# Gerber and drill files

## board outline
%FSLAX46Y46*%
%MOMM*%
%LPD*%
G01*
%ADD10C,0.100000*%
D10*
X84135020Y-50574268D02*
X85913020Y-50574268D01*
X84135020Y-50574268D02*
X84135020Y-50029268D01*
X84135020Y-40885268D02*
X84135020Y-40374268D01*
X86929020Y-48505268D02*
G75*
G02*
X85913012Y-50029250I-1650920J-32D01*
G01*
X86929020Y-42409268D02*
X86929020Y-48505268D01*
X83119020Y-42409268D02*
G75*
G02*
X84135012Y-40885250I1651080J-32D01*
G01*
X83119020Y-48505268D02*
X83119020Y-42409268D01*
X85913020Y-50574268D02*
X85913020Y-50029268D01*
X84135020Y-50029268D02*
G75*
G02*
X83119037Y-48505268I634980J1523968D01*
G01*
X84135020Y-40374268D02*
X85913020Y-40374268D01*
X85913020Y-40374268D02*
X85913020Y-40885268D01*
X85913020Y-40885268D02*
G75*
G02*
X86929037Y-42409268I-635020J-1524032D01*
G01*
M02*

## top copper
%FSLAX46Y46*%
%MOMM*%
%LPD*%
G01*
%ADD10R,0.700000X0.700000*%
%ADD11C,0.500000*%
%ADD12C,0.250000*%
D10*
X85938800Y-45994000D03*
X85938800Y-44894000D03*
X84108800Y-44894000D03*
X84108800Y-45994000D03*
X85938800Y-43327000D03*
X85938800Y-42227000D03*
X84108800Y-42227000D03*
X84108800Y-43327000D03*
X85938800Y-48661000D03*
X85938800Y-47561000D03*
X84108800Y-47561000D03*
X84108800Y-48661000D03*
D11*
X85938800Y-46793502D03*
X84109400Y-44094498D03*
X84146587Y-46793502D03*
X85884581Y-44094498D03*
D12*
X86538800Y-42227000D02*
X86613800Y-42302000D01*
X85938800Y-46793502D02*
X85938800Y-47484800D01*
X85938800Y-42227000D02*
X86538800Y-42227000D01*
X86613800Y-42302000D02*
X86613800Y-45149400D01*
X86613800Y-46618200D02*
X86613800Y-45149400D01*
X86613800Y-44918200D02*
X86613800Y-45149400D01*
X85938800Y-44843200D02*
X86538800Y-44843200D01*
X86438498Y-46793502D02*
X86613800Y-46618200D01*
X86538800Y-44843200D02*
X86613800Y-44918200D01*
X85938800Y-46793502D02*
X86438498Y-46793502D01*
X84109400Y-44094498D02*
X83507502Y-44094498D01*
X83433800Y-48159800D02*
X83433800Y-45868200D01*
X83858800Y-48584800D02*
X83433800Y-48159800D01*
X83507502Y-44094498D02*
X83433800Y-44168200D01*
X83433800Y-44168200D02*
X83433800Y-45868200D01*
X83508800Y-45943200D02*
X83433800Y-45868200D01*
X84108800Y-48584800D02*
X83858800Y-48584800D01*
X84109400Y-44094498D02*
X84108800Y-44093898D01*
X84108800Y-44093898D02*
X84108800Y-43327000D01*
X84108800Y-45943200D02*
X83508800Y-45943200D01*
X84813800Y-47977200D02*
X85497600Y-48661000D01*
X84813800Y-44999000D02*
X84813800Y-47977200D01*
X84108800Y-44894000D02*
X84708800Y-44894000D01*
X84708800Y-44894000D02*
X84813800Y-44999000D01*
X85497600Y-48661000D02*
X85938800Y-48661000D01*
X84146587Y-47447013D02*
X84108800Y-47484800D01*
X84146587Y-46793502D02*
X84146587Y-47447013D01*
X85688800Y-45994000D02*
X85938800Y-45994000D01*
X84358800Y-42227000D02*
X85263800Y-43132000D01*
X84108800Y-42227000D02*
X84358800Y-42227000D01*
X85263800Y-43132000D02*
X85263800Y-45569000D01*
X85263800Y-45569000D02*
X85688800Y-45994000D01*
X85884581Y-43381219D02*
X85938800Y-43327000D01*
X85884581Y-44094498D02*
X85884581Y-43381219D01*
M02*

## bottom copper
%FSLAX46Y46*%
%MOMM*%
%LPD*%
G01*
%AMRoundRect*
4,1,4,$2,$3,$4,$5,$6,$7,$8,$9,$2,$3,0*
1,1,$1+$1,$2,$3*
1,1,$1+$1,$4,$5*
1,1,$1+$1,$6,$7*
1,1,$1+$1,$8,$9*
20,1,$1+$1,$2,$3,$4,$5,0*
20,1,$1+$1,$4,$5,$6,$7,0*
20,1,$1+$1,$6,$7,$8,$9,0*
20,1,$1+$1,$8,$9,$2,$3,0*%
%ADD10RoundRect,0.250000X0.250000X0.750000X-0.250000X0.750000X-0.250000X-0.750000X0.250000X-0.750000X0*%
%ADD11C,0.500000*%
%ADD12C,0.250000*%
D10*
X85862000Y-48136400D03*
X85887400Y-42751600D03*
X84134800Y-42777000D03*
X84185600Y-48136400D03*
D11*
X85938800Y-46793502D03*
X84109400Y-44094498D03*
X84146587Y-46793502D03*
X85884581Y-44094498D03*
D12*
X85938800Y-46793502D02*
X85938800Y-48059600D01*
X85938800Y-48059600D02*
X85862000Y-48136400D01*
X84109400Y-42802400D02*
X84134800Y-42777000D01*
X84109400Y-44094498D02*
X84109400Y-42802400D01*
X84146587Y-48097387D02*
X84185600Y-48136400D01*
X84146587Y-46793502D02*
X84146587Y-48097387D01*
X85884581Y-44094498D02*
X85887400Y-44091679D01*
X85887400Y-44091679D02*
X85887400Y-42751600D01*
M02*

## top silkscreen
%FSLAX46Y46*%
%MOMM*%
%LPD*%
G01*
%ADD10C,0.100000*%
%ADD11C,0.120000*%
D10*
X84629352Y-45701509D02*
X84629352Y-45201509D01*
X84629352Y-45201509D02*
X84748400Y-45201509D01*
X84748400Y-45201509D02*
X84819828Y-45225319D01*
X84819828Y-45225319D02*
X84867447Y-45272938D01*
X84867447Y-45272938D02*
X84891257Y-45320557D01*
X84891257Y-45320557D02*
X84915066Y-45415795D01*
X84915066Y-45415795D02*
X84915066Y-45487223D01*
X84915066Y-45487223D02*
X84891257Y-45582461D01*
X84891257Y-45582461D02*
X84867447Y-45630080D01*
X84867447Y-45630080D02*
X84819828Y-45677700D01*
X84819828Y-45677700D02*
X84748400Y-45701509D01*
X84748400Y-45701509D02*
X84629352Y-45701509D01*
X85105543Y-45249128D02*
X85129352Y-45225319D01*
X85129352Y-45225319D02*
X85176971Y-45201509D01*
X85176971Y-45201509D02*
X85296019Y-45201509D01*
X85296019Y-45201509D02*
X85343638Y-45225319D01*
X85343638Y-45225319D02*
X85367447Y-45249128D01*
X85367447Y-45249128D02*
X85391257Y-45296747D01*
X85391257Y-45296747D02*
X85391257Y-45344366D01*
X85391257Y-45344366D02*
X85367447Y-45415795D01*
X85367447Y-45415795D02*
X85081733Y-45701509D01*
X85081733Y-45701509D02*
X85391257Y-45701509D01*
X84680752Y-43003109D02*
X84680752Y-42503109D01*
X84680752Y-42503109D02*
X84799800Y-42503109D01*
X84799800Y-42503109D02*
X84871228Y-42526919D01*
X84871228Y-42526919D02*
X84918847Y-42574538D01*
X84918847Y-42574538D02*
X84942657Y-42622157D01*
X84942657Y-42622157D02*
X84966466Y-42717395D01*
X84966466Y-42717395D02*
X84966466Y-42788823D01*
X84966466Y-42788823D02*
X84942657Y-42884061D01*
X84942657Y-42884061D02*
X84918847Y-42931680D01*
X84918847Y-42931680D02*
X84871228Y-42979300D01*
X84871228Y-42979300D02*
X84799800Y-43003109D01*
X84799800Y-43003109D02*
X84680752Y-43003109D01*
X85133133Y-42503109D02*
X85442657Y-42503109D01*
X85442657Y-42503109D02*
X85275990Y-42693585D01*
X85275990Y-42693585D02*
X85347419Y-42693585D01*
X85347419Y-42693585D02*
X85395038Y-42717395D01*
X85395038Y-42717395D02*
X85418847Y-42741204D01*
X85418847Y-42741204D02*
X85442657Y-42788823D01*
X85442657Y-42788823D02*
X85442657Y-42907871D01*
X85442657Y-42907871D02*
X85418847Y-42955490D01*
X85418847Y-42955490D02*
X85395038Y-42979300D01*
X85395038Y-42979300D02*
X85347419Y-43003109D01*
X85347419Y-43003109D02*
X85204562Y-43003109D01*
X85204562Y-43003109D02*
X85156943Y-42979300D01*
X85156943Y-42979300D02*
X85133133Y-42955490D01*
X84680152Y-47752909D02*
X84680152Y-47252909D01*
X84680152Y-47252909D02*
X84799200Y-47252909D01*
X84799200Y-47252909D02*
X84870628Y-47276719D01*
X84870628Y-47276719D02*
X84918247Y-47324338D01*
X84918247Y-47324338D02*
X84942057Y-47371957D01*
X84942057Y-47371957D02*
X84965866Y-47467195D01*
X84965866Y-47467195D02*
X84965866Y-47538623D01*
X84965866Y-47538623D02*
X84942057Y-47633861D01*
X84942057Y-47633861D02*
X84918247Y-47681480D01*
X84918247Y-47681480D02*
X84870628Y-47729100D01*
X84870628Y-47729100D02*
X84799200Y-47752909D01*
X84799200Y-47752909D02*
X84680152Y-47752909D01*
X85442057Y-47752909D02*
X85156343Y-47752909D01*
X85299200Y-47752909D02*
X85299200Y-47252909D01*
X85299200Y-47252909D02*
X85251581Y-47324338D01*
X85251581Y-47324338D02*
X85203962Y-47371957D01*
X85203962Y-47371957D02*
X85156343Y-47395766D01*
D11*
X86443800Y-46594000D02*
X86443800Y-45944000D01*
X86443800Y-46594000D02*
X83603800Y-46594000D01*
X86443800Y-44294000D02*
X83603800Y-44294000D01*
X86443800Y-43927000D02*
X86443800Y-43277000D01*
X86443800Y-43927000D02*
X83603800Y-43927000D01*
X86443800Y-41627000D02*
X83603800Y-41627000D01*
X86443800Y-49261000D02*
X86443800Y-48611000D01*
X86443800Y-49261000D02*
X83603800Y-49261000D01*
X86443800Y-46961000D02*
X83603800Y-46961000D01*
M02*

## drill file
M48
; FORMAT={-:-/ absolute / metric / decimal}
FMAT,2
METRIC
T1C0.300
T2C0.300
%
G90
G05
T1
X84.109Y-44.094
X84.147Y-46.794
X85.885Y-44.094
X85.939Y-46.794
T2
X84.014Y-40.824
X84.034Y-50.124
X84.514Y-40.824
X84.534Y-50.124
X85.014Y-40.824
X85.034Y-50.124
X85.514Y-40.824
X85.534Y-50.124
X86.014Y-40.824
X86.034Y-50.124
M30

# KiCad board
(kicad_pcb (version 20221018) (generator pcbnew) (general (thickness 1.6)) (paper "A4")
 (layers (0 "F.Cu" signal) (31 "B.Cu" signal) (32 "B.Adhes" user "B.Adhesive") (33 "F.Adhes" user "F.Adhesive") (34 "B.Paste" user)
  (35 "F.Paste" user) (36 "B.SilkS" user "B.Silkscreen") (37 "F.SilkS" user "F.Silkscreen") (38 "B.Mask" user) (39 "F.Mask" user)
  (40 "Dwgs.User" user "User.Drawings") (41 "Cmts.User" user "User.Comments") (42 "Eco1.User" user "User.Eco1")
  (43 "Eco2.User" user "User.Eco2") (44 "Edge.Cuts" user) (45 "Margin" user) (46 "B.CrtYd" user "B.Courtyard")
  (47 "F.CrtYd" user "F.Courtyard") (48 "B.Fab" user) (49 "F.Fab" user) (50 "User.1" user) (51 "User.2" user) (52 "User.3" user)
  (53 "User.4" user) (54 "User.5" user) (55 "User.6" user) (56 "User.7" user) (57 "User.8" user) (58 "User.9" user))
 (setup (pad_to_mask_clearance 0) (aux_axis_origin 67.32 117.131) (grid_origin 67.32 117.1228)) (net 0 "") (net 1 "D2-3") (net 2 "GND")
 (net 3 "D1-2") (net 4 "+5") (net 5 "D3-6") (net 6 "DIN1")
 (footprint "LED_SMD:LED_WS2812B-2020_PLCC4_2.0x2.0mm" (layer "F.Cu") (at 85.0238 45.444 180)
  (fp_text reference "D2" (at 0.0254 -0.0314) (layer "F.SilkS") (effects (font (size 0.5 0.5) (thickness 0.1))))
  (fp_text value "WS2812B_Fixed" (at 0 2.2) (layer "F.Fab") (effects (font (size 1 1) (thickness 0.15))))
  (fp_line (start -1.42 -1.15) (end -1.42 -0.5) (stroke (width 0.12) (type solid)) (layer "F.SilkS"))
  (fp_line (start -1.42 -1.15) (end 1.42 -1.15) (stroke (width 0.12) (type solid)) (layer "F.SilkS"))
  (fp_line (start -1.42 1.15) (end 1.42 1.15) (stroke (width 0.12) (type solid)) (layer "F.SilkS"))
  (pad "1" smd rect (at -0.915 -0.55 180) (size 0.7 0.7) (layers "F.Cu" "F.Paste" "F.Mask") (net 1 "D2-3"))
  (pad "2" smd rect (at -0.915 0.55 180) (size 0.7 0.7) (layers "F.Cu" "F.Paste" "F.Mask") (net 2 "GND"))
  (pad "3" smd rect (at 0.915 0.55 180) (size 0.7 0.7) (layers "F.Cu" "F.Paste" "F.Mask") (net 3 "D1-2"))
  (pad "4" smd rect (at 0.915 -0.55 180) (size 0.7 0.7) (layers "F.Cu" "F.Paste" "F.Mask") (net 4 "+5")))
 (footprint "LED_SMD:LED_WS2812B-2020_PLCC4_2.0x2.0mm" (layer "F.Cu") (at 85.0238 42.777 180)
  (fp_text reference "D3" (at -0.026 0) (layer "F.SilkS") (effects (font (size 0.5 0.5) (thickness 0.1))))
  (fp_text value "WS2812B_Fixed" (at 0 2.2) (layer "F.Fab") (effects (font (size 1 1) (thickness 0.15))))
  (fp_line (start -1.42 -1.15) (end -1.42 -0.5) (stroke (width 0.12) (type solid)) (layer "F.SilkS"))
  (fp_line (start -1.42 -1.15) (end 1.42 -1.15) (stroke (width 0.12) (type solid)) (layer "F.SilkS"))
  (fp_line (start -1.42 1.15) (end 1.42 1.15) (stroke (width 0.12) (type solid)) (layer "F.SilkS"))
  (pad "1" smd rect (at -0.915 -0.55 180) (size 0.7 0.7) (layers "F.Cu" "F.Paste" "F.Mask") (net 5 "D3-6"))
  (pad "2" smd rect (at -0.915 0.55 180) (size 0.7 0.7) (layers "F.Cu" "F.Paste" "F.Mask") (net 2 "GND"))
  (pad "3" smd rect (at 0.915 0.55 180) (size 0.7 0.7) (layers "F.Cu" "F.Paste" "F.Mask") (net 1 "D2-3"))
  (pad "4" smd rect (at 0.915 -0.55 180) (size 0.7 0.7) (layers "F.Cu" "F.Paste" "F.Mask") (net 4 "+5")))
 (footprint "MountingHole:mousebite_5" (layer "F.Cu") (at 85.03362 50.124268)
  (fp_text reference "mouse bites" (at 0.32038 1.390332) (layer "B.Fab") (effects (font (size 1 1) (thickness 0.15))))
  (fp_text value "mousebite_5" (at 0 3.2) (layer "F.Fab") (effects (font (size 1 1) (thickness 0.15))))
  (pad "" np_thru_hole circle (at -1 0) (size 0.3 0.3) (drill 0.3) (layers "F&B.Cu" "*.Mask"))
  (pad "" np_thru_hole circle (at -0.5 0) (size 0.3 0.3) (drill 0.3) (layers "F&B.Cu" "*.Mask"))
  (pad "" np_thru_hole circle (at 0 0) (size 0.3 0.3) (drill 0.3) (layers "F&B.Cu" "*.Mask"))
  (pad "" np_thru_hole circle (at 0.5 0) (size 0.3 0.3) (drill 0.3) (layers "F&B.Cu" "*.Mask"))
  (pad "" np_thru_hole circle (at 1 0) (size 0.3 0.3) (drill 0.3) (layers "F&B.Cu" "*.Mask")))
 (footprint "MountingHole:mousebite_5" (layer "F.Cu") (at 85.01362 40.824268)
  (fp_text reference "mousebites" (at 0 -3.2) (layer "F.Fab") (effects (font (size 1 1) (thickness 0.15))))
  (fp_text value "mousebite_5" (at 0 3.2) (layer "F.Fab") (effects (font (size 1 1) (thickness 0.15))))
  (pad "" np_thru_hole circle (at -1 0) (size 0.3 0.3) (drill 0.3) (layers "F&B.Cu" "*.Mask"))
  (pad "" np_thru_hole circle (at -0.5 0) (size 0.3 0.3) (drill 0.3) (layers "F&B.Cu" "*.Mask"))
  (pad "" np_thru_hole circle (at 0 0) (size 0.3 0.3) (drill 0.3) (layers "F&B.Cu" "*.Mask"))
  (pad "" np_thru_hole circle (at 0.5 0) (size 0.3 0.3) (drill 0.3) (layers "F&B.Cu" "*.Mask"))
  (pad "" np_thru_hole circle (at 1 0) (size 0.3 0.3) (drill 0.3) (layers "F&B.Cu" "*.Mask")))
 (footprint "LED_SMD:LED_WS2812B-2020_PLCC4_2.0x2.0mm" (layer "F.Cu") (at 85.0238 48.111 180)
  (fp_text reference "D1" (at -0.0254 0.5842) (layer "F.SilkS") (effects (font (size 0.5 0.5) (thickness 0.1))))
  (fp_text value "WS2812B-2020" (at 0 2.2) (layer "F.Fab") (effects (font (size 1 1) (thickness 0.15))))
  (fp_line (start -1.42 -1.15) (end -1.42 -0.5) (stroke (width 0.12) (type solid)) (layer "F.SilkS"))
  (fp_line (start -1.42 -1.15) (end 1.42 -1.15) (stroke (width 0.12) (type solid)) (layer "F.SilkS"))
  (fp_line (start -1.42 1.15) (end 1.42 1.15) (stroke (width 0.12) (type solid)) (layer "F.SilkS"))
  (pad "1" smd rect (at -0.915 -0.55 180) (size 0.7 0.7) (layers "F.Cu" "F.Paste" "F.Mask") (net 3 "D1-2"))
  (pad "2" smd rect (at -0.915 0.55 180) (size 0.7 0.7) (layers "F.Cu" "F.Paste" "F.Mask") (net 2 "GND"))
  (pad "3" smd rect (at 0.915 0.55 180) (size 0.7 0.7) (layers "F.Cu" "F.Paste" "F.Mask") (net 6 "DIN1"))
  (pad "4" smd rect (at 0.915 -0.55 180) (size 0.7 0.7) (layers "F.Cu" "F.Paste" "F.Mask") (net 4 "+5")))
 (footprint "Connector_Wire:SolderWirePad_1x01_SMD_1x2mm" (layer "B.Cu") (at 85.862 48.1364 180)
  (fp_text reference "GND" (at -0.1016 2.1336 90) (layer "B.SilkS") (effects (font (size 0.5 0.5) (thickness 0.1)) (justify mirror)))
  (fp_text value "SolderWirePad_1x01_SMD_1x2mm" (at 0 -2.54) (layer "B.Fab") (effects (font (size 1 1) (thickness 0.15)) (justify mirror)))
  (pad "1" smd roundrect (at 0 0 180) (size 1 2) (layers "B.Cu" "B.Paste" "B.Mask") (roundrect_rratio 0.25) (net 2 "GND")))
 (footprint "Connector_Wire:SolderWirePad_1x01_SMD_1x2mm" (layer "B.Cu") (at 85.8874 42.7516 180)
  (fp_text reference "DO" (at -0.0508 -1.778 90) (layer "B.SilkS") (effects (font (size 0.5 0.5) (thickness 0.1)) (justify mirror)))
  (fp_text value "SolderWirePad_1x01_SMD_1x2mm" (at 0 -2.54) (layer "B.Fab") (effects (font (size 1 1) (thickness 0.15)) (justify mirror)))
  (pad "1" smd roundrect (at 0 0 180) (size 1 2) (layers "B.Cu" "B.Paste" "B.Mask") (roundrect_rratio 0.25) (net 5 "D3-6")))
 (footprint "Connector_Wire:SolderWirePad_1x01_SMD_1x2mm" (layer "B.Cu") (at 84.1348 42.777 180)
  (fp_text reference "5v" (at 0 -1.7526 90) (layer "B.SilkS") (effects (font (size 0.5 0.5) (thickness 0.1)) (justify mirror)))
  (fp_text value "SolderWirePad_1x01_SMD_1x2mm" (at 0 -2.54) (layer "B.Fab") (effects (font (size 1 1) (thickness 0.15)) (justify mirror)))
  (pad "4" smd roundrect (at 0 0 180) (size 1 2) (layers "B.Cu" "B.Paste" "B.Mask") (roundrect_rratio 0.25) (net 4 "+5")))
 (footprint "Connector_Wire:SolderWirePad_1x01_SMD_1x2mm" (layer "B.Cu") (at 84.1856 48.1364 180)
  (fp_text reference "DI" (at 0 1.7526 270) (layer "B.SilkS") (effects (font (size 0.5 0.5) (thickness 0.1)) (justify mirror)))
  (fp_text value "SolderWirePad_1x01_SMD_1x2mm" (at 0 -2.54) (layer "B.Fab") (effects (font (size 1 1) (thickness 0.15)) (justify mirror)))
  (pad "3" smd roundrect (at 0 0 180) (size 1 2) (layers "B.Cu" "B.Paste" "B.Mask") (roundrect_rratio 0.25) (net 6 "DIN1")))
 (gr_line (start 84.13502 50.574268) (end 85.91302 50.574268) (stroke (width 0.1) (type solid)) (layer "Edge.Cuts"))
 (gr_line (start 84.13502 50.574268) (end 84.13502 50.029268) (stroke (width 0.1) (type solid)) (layer "Edge.Cuts"))
 (gr_line (start 84.13502 40.885268) (end 84.13502 40.374268) (stroke (width 0.1) (type solid)) (layer "Edge.Cuts"))
 (gr_arc (start 86.92902 48.505268) (mid 86.651749 49.421087) (end 85.91302 50.029268) (stroke (width 0.1) (type solid)) (layer "Edge.Cuts"))
 (gr_line (start 86.92902 42.409268) (end 86.92902 48.505268) (stroke (width 0.1) (type solid)) (layer "Edge.Cuts"))
 (gr_arc (start 83.11902 42.409268) (mid 83.396319 41.493467) (end 84.13502 40.885268) (stroke (width 0.1) (type solid)) (layer "Edge.Cuts"))
 (gr_line (start 83.11902 48.505268) (end 83.11902 42.409268) (stroke (width 0.1) (type solid)) (layer "Edge.Cuts"))
 (gr_line (start 85.91302 50.574268) (end 85.91302 50.029268) (stroke (width 0.1) (type solid)) (layer "Edge.Cuts"))
 (gr_arc (start 84.13502 50.029268) (mid 83.396296 49.421083) (end 83.11902 48.505268) (stroke (width 0.1) (type solid)) (layer "Edge.Cuts"))
 (gr_line (start 84.13502 40.374268) (end 85.91302 40.374268) (stroke (width 0.1) (type solid)) (layer "Edge.Cuts"))
 (gr_line (start 85.91302 40.374268) (end 85.91302 40.885268) (stroke (width 0.1) (type solid)) (layer "Edge.Cuts"))
 (gr_arc (start 85.91302 40.885268) (mid 86.651727 41.493463) (end 86.92902 42.409268) (stroke (width 0.1) (type solid)) (layer "Edge.Cuts"))
 (segment (start 86.5388 42.227) (end 86.6138 42.302) (width 0.25) (layer "F.Cu") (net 2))
 (segment (start 85.9388 46.793502) (end 85.9388 47.4848) (width 0.25) (layer "F.Cu") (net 2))
 (segment (start 85.9388 42.227) (end 86.5388 42.227) (width 0.25) (layer "F.Cu") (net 2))
 (segment (start 86.6138 42.302) (end 86.6138 45.1494) (width 0.25) (layer "F.Cu") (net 2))
 (segment (start 86.6138 46.6182) (end 86.6138 45.1494) (width 0.25) (layer "F.Cu") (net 2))
 (segment (start 86.6138 44.9182) (end 86.6138 45.1494) (width 0.25) (layer "F.Cu") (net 2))
 (segment (start 85.9388 44.8432) (end 86.5388 44.8432) (width 0.25) (layer "F.Cu") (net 2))
 (segment (start 86.438498 46.793502) (end 86.6138 46.6182) (width 0.25) (layer "F.Cu") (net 2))
 (segment (start 86.5388 44.8432) (end 86.6138 44.9182) (width 0.25) (layer "F.Cu") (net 2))
 (segment (start 85.9388 46.793502) (end 86.438498 46.793502) (width 0.25) (layer "F.Cu") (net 2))
 (via (at 85.9388 46.793502) (size 0.5) (drill 0.3) (layers "F.Cu" "B.Cu") (free) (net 2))
 (segment (start 85.9388 46.793502) (end 85.9388 48.0596) (width 0.25) (layer "B.Cu") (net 2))
 (segment (start 85.9388 48.0596) (end 85.862 48.1364) (width 0.25) (layer "B.Cu") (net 2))
 (segment (start 84.1094 44.094498) (end 83.507502 44.094498) (width 0.25) (layer "F.Cu") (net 4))
 (segment (start 83.4338 48.1598) (end 83.4338 45.8682) (width 0.25) (layer "F.Cu") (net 4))
 (segment (start 83.8588 48.5848) (end 83.4338 48.1598) (width 0.25) (layer "F.Cu") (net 4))
 (segment (start 83.507502 44.094498) (end 83.4338 44.1682) (width 0.25) (layer "F.Cu") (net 4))
 (segment (start 83.4338 44.1682) (end 83.4338 45.8682) (width 0.25) (layer "F.Cu") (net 4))
 (segment (start 83.5088 45.9432) (end 83.4338 45.8682) (width 0.25) (layer "F.Cu") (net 4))
 (segment (start 84.1088 48.5848) (end 83.8588 48.5848) (width 0.25) (layer "F.Cu") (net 4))
 (segment (start 84.1094 44.094498) (end 84.1088 44.093898) (width 0.25) (layer "F.Cu") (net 4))
 (segment (start 84.1088 44.093898) (end 84.1088 43.327) (width 0.25) (layer "F.Cu") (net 4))
 (segment (start 84.1088 45.9432) (end 83.5088 45.9432) (width 0.25) (layer "F.Cu") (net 4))
 (via (at 84.1094 44.094498) (size 0.5) (drill 0.3) (layers "F.Cu" "B.Cu") (free) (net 4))
 (segment (start 84.1094 42.8024) (end 84.1348 42.777) (width 0.25) (layer "B.Cu") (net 4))
 (segment (start 84.1094 44.094498) (end 84.1094 42.8024) (width 0.25) (layer "B.Cu") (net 4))
 (segment (start 84.8138 47.9772) (end 85.4976 48.661) (width 0.25) (layer "F.Cu") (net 3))
 (segment (start 84.8138 44.999) (end 84.8138 47.9772) (width 0.25) (layer "F.Cu") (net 3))
 (segment (start 84.1088 44.894) (end 84.7088 44.894) (width 0.25) (layer "F.Cu") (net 3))
 (segment (start 84.7088 44.894) (end 84.8138 44.999) (width 0.25) (layer "F.Cu") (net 3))
 (segment (start 85.4976 48.661) (end 85.9388 48.661) (width 0.25) (layer "F.Cu") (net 3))
 (segment (start 84.146587 47.447013) (end 84.1088 47.4848) (width 0.25) (layer "F.Cu") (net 6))
 (segment (start 84.146587 46.793502) (end 84.146587 47.447013) (width 0.25) (layer "F.Cu") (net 6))
 (via (at 84.146587 46.793502) (size 0.5) (drill 0.3) (layers "F.Cu" "B.Cu") (free) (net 6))
 (segment (start 84.146587 48.097387) (end 84.1856 48.1364) (width 0.25) (layer "B.Cu") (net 6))
 (segment (start 84.146587 46.793502) (end 84.146587 48.097387) (width 0.25) (layer "B.Cu") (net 6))
 (segment (start 85.6888 45.994) (end 85.9388 45.994) (width 0.25) (layer "F.Cu") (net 1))
 (segment (start 84.3588 42.227) (end 85.2638 43.132) (width 0.25) (layer "F.Cu") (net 1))
 (segment (start 84.1088 42.227) (end 84.3588 42.227) (width 0.25) (layer "F.Cu") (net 1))
 (segment (start 85.2638 43.132) (end 85.2638 45.569) (width 0.25) (layer "F.Cu") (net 1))
 (segment (start 85.2638 45.569) (end 85.6888 45.994) (width 0.25) (layer "F.Cu") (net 1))
 (segment (start 85.884581 43.381219) (end 85.9388 43.327) (width 0.25) (layer "F.Cu") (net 5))
 (segment (start 85.884581 44.094498) (end 85.884581 43.381219) (width 0.25) (layer "F.Cu") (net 5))
 (via (at 85.884581 44.094498) (size 0.5) (drill 0.3) (layers "F.Cu" "B.Cu") (free) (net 5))
 (segment (start 85.884581 44.094498) (end 85.8874 44.091679) (width 0.25) (layer "B.Cu") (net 5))
 (segment (start 85.8874 44.091679) (end 85.8874 42.7516) (width 0.25) (layer "B.Cu") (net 5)))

